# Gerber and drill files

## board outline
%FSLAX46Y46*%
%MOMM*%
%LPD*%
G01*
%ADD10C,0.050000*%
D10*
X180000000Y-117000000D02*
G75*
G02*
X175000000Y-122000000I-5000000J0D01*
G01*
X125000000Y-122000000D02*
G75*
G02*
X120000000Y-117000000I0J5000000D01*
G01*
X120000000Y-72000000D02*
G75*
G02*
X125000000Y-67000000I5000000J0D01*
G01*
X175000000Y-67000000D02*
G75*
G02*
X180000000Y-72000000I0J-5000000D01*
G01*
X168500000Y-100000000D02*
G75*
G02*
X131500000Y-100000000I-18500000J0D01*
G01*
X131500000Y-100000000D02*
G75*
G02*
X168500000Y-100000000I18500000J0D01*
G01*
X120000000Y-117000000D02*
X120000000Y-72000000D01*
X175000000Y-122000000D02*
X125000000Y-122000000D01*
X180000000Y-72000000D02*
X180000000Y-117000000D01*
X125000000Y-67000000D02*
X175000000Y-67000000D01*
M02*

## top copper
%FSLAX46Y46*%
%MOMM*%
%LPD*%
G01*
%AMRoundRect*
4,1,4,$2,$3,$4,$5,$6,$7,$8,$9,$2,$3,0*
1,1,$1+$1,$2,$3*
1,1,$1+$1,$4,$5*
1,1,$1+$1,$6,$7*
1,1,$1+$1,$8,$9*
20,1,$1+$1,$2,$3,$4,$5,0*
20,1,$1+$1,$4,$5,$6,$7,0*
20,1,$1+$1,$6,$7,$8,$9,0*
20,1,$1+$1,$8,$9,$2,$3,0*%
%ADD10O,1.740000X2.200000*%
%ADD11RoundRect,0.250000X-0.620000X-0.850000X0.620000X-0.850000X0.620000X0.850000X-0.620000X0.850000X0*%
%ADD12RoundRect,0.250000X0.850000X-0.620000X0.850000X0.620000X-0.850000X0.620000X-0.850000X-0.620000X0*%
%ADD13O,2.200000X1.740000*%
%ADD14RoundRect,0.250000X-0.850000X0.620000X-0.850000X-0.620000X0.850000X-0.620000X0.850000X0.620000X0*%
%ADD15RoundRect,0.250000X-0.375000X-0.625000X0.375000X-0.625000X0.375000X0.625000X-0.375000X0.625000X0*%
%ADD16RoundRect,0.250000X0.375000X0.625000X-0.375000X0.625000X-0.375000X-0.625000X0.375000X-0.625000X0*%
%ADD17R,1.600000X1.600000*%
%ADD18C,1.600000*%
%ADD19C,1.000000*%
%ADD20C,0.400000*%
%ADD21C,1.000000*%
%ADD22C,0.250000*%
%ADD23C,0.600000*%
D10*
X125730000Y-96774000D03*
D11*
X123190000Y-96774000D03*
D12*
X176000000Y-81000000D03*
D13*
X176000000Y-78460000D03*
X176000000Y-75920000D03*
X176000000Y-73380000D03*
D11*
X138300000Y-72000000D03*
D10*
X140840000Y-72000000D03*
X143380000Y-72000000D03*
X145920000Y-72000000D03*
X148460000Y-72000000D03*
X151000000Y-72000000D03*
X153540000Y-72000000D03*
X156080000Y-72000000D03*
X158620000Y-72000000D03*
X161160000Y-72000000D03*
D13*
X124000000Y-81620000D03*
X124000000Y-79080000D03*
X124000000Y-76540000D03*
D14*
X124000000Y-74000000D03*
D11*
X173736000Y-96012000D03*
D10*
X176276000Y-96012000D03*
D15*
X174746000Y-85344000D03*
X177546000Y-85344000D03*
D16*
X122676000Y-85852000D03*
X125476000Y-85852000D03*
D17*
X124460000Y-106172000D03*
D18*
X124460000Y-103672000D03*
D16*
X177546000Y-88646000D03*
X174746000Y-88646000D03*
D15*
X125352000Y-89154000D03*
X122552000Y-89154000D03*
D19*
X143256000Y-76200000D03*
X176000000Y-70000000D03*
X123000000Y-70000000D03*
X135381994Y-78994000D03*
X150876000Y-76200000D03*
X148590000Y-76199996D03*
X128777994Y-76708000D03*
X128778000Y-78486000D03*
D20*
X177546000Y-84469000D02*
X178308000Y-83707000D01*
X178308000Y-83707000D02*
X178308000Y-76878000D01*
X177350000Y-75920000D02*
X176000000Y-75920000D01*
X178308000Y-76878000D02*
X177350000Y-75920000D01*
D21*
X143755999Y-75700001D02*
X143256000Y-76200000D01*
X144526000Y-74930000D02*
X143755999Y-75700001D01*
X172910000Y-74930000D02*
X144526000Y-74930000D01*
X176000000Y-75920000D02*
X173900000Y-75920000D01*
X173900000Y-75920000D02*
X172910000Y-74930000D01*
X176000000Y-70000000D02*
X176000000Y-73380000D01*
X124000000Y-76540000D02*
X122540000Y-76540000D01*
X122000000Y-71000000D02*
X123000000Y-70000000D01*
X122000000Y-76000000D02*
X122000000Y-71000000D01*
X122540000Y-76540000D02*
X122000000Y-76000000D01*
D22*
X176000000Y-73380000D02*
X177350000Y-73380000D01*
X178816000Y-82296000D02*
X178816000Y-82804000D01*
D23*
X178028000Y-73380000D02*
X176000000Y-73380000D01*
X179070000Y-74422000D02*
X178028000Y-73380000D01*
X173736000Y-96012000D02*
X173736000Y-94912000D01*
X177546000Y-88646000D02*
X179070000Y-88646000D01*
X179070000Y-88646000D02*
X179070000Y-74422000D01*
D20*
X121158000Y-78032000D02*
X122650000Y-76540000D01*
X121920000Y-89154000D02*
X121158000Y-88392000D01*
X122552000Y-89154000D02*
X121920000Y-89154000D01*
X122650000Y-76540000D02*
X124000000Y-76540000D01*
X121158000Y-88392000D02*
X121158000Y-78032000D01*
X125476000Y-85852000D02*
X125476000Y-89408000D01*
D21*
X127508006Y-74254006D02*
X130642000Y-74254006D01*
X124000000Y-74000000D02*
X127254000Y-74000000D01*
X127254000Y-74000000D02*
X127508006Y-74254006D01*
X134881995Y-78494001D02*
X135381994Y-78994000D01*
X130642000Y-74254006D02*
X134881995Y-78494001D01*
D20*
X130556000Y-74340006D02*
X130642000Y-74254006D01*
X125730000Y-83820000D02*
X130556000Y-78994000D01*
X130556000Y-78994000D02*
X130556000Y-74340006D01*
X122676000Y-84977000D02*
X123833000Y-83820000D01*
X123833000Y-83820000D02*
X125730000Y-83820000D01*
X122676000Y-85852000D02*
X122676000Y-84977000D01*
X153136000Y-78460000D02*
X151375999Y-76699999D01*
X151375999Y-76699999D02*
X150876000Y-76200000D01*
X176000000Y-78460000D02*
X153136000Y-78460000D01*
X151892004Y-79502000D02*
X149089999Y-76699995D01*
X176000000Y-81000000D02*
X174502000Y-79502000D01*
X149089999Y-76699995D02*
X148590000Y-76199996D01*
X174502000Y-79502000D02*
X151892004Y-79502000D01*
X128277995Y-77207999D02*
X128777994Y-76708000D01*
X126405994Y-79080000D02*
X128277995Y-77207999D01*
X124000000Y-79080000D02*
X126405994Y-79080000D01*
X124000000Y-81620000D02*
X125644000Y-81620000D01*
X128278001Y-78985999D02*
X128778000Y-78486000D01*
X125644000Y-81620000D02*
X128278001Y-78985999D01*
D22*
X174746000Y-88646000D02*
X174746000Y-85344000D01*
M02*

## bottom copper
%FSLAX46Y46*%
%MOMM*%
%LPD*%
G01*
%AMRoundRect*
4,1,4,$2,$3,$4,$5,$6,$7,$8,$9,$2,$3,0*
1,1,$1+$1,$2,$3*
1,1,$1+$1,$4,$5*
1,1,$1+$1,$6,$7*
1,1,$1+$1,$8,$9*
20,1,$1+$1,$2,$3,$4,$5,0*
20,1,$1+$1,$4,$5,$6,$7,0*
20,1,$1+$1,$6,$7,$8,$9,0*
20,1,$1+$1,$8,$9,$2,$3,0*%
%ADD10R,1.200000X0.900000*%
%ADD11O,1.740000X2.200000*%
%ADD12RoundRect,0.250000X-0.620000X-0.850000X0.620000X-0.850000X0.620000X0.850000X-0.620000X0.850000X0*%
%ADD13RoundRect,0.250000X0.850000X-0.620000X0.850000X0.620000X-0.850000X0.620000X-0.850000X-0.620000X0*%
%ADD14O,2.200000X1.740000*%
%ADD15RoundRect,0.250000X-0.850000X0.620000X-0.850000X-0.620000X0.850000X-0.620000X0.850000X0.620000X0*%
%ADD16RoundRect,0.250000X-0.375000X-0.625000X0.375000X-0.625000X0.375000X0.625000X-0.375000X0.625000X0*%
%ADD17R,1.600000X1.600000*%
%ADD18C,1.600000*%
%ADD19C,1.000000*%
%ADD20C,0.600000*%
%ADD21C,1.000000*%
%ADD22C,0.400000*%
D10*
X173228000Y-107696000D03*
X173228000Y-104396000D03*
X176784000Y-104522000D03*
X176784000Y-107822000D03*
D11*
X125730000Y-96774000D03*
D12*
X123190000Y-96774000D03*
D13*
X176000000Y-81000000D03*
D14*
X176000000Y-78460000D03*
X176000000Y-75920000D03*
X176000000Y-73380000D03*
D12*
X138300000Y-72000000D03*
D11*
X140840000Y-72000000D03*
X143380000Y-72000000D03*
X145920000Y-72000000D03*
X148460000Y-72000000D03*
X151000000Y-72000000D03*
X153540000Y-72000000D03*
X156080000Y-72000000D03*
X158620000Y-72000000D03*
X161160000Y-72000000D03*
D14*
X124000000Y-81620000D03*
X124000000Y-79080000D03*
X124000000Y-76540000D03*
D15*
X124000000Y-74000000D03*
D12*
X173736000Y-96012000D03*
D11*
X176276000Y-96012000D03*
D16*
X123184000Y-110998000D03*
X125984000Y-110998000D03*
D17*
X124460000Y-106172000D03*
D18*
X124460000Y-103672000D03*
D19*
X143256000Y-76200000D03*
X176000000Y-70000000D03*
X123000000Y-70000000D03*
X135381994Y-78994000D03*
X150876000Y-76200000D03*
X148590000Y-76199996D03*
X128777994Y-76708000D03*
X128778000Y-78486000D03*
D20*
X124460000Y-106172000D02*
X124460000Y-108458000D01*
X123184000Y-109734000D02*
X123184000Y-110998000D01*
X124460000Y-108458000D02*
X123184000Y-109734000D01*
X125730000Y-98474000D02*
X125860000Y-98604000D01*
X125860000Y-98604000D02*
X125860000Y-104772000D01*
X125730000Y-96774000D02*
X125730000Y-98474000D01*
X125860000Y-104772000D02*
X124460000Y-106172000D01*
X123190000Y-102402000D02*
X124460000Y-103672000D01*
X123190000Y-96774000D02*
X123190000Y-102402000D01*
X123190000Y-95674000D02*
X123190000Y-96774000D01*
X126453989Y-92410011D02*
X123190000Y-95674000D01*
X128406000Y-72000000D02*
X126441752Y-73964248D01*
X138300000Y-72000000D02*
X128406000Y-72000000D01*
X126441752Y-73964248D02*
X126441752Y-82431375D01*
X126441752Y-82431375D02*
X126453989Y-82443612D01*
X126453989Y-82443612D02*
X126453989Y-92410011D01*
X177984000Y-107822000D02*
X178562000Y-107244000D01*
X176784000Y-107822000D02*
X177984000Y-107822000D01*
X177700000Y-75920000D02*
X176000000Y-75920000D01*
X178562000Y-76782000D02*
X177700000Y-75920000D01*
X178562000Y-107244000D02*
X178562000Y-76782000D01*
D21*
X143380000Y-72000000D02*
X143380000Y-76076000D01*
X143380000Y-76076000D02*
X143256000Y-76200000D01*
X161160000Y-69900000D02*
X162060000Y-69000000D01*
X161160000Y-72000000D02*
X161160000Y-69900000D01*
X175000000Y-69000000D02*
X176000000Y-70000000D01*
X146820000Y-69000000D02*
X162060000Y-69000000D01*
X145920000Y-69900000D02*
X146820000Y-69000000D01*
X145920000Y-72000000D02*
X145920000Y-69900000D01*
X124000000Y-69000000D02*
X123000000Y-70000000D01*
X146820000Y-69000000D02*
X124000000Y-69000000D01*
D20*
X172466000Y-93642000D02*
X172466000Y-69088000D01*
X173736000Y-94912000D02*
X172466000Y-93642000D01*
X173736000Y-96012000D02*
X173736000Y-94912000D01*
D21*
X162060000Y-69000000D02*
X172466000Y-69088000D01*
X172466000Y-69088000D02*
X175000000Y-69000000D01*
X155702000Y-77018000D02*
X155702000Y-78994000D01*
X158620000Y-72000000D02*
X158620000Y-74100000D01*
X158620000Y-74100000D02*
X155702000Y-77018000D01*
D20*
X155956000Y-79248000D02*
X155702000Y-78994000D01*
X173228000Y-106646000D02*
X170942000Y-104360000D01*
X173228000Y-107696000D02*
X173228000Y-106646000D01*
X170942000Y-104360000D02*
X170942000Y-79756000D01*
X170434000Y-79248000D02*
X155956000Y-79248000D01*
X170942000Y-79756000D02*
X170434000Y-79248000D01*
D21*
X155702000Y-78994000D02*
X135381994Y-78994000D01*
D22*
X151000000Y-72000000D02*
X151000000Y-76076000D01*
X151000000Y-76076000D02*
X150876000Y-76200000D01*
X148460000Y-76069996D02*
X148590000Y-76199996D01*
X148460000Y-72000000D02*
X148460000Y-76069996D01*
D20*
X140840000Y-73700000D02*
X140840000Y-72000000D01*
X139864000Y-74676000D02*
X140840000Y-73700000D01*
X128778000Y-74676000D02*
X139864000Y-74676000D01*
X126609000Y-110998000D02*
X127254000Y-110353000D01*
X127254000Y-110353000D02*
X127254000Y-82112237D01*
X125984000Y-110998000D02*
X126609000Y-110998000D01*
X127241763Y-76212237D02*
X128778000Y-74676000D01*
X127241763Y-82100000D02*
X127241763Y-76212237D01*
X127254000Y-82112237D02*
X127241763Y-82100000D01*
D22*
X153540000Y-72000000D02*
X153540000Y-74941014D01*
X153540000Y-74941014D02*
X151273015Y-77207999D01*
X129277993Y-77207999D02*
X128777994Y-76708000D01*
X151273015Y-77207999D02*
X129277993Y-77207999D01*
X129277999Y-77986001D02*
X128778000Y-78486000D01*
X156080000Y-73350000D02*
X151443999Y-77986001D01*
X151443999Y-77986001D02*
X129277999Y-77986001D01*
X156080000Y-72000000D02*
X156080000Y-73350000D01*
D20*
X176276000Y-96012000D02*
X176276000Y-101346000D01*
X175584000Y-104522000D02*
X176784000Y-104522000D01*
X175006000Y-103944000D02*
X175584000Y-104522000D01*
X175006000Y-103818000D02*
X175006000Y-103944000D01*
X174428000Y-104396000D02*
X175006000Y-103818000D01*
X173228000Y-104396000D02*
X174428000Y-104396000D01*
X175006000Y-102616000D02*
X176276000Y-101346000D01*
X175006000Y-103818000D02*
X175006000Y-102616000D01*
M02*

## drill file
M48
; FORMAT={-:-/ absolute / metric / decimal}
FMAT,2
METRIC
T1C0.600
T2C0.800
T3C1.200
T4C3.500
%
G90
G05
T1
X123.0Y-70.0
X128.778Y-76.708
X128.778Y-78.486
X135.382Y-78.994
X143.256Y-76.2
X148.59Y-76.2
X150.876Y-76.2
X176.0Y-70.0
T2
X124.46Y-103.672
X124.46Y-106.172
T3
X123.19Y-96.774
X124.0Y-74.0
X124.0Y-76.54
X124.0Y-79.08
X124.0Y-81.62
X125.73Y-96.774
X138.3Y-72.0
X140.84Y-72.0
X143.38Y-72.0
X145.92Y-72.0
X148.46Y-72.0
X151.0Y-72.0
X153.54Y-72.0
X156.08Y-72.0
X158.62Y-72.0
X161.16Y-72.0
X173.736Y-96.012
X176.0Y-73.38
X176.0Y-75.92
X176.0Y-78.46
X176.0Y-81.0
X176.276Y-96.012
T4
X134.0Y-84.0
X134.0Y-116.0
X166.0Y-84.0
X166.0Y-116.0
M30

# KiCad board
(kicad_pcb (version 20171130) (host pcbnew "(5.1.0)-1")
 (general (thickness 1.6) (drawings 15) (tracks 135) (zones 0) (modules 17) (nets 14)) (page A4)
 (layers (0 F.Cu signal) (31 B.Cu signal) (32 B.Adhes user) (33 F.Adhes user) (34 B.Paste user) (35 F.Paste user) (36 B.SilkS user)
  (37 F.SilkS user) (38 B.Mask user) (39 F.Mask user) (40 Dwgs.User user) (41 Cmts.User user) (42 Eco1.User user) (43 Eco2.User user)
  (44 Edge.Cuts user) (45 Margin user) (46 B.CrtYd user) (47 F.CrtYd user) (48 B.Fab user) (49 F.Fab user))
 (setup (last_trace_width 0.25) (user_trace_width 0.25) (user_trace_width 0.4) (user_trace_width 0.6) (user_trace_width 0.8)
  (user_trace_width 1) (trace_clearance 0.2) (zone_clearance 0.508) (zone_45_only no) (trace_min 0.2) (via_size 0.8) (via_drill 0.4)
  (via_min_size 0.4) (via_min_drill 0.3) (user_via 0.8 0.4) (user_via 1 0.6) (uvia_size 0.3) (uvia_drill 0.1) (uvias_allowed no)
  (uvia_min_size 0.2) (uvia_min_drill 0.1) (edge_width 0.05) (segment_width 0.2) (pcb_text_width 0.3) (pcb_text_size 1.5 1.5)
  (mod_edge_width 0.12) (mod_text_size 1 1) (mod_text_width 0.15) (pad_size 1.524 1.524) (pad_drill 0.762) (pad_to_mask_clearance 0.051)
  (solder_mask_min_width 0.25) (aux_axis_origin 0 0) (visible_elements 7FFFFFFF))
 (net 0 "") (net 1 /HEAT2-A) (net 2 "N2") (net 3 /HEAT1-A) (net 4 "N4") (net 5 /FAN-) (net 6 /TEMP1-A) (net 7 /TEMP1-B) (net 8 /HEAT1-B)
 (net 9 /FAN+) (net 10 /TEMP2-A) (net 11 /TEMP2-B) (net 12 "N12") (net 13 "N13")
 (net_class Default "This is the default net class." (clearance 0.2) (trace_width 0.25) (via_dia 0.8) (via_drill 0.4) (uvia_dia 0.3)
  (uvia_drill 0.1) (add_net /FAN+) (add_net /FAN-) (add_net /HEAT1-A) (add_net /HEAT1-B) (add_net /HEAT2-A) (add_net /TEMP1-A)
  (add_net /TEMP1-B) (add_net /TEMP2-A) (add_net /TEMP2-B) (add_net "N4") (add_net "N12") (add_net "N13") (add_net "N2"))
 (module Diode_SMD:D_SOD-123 (layer B.Cu) (at 173.228 106.046 270)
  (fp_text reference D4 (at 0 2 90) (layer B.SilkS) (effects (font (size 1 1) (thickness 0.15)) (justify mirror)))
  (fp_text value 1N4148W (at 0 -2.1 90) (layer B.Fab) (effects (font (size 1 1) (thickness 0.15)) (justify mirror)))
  (pad 2 smd rect (at 1.65 0 270) (size 0.9 1.2) (layers B.Cu B.Paste B.Mask) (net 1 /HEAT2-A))
  (pad 1 smd rect (at -1.65 0 270) (size 0.9 1.2) (layers B.Cu B.Paste B.Mask) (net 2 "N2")))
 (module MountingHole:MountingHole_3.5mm (layer F.Cu) (at 134 116)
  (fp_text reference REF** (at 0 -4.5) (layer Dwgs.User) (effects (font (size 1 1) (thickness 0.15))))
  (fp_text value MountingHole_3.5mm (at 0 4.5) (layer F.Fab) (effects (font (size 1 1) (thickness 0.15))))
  (pad 1 np_thru_hole circle (at 0 0) (size 3.5 3.5) (drill 3.5) (layers *.Cu *.Mask)))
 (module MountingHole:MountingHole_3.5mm (layer F.Cu) (at 166 116)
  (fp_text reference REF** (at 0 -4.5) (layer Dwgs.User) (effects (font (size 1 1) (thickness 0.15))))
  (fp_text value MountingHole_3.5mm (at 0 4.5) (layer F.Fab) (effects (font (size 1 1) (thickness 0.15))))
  (pad 1 np_thru_hole circle (at 0 0) (size 3.5 3.5) (drill 3.5) (layers *.Cu *.Mask)))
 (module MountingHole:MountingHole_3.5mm (layer F.Cu) (at 166 84)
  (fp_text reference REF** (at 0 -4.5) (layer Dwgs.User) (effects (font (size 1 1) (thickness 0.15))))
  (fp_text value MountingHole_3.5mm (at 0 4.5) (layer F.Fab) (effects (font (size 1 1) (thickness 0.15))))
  (pad 1 np_thru_hole circle (at 0 0) (size 3.5 3.5) (drill 3.5) (layers *.Cu *.Mask)))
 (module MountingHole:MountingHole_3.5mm (layer F.Cu) (at 134 84)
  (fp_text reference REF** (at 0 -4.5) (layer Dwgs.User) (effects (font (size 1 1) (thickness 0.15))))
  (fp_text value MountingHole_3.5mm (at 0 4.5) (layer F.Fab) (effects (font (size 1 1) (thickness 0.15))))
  (pad 1 np_thru_hole circle (at 0 0) (size 3.5 3.5) (drill 3.5) (layers *.Cu *.Mask)))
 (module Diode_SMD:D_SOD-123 (layer B.Cu) (at 176.784 106.172 270)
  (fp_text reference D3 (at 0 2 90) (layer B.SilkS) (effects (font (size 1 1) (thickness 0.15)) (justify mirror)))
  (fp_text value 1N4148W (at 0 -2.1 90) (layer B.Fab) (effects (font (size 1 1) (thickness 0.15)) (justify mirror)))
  (pad 1 smd rect (at -1.65 0 270) (size 0.9 1.2) (layers B.Cu B.Paste B.Mask) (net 2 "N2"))
  (pad 2 smd rect (at 1.65 0 270) (size 0.9 1.2) (layers B.Cu B.Paste B.Mask) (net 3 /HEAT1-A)))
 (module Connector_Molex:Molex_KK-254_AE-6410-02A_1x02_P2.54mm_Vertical (layer F.Cu) (at 123.19 96.774)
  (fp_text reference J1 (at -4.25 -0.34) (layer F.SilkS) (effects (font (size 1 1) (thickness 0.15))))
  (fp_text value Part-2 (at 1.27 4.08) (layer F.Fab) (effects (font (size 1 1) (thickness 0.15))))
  (pad 2 thru_hole oval (at 2.54 0) (size 1.74 2.2) (drill 1.2) (layers *.Cu *.Mask) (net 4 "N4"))
  (pad 1 thru_hole roundrect (at 0 0) (size 1.74 2.2) (drill 1.2) (layers *.Cu *.Mask) (roundrect_rratio 0.143678) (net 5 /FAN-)))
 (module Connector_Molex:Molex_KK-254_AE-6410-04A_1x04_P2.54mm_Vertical (layer B.Cu) (at 176 81 90)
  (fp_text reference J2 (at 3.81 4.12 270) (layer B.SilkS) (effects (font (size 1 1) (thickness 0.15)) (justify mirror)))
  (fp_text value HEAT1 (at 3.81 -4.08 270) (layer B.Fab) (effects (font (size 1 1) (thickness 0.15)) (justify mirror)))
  (pad 1 thru_hole roundrect (at 0 0 90) (size 1.74 2.2) (drill 1.2) (layers *.Cu *.Mask) (roundrect_rratio 0.143678) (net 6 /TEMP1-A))
  (pad 2 thru_hole oval (at 2.54 0 90) (size 1.74 2.2) (drill 1.2) (layers *.Cu *.Mask) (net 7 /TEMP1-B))
  (pad 3 thru_hole oval (at 5.08 0 90) (size 1.74 2.2) (drill 1.2) (layers *.Cu *.Mask) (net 3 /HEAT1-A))
  (pad 4 thru_hole oval (at 7.62 0 90) (size 1.74 2.2) (drill 1.2) (layers *.Cu *.Mask) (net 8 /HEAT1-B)))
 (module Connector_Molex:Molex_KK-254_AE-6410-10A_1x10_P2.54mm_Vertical (layer F.Cu) (at 138.3 72)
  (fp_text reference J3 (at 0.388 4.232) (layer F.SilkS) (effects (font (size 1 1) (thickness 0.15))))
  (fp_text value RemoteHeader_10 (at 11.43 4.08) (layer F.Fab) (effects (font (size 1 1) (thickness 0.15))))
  (pad 1 thru_hole roundrect (at 0 0) (size 1.74 2.2) (drill 1.2) (layers *.Cu *.Mask) (roundrect_rratio 0.143678) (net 5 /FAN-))
  (pad 2 thru_hole oval (at 2.54 0) (size 1.74 2.2) (drill 1.2) (layers *.Cu *.Mask) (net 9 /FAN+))
  (pad 3 thru_hole oval (at 5.08 0) (size 1.74 2.2) (drill 1.2) (layers *.Cu *.Mask) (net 3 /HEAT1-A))
  (pad 4 thru_hole oval (at 7.62 0) (size 1.74 2.2) (drill 1.2) (layers *.Cu *.Mask) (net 8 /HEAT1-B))
  (pad 5 thru_hole oval (at 10.16 0) (size 1.74 2.2) (drill 1.2) (layers *.Cu *.Mask) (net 6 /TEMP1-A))
  (pad 6 thru_hole oval (at 12.7 0) (size 1.74 2.2) (drill 1.2) (layers *.Cu *.Mask) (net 7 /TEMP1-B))
  (pad 7 thru_hole oval (at 15.24 0) (size 1.74 2.2) (drill 1.2) (layers *.Cu *.Mask) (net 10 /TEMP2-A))
  (pad 8 thru_hole oval (at 17.78 0) (size 1.74 2.2) (drill 1.2) (layers *.Cu *.Mask) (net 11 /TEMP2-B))
  (pad 9 thru_hole oval (at 20.32 0) (size 1.74 2.2) (drill 1.2) (layers *.Cu *.Mask) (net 1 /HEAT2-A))
  (pad 10 thru_hole oval (at 22.86 0) (size 1.74 2.2) (drill 1.2) (layers *.Cu *.Mask) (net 8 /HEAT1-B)))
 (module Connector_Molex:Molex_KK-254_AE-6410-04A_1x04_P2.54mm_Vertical (layer B.Cu) (at 124 74 270)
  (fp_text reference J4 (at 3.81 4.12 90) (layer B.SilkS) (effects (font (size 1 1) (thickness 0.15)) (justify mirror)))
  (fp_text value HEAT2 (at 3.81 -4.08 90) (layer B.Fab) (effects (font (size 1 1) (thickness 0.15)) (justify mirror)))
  (pad 4 thru_hole oval (at 7.62 0 270) (size 1.74 2.2) (drill 1.2) (layers *.Cu *.Mask) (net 11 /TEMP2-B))
  (pad 3 thru_hole oval (at 5.08 0 270) (size 1.74 2.2) (drill 1.2) (layers *.Cu *.Mask) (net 10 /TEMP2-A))
  (pad 2 thru_hole oval (at 2.54 0 270) (size 1.74 2.2) (drill 1.2) (layers *.Cu *.Mask) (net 8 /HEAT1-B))
  (pad 1 thru_hole roundrect (at 0 0 270) (size 1.74 2.2) (drill 1.2) (layers *.Cu *.Mask) (roundrect_rratio 0.143678) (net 1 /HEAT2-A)))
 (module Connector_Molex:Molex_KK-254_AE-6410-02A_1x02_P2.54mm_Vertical (layer F.Cu) (at 173.736 96.012)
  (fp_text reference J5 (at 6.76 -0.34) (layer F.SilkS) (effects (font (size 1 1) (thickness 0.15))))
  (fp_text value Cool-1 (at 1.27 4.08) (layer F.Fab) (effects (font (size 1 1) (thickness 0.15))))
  (pad 1 thru_hole roundrect (at 0 0) (size 1.74 2.2) (drill 1.2) (layers *.Cu *.Mask) (roundrect_rratio 0.143678) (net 8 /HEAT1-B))
  (pad 2 thru_hole oval (at 2.54 0) (size 1.74 2.2) (drill 1.2) (layers *.Cu *.Mask) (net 2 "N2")))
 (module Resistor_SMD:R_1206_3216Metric (layer F.Cu) (at 176.146 85.344)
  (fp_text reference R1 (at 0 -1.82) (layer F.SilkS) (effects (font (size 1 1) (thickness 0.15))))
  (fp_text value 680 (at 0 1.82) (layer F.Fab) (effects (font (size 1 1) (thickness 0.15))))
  (pad 1 smd roundrect (at -1.4 0) (size 1.25 1.75) (layers F.Cu F.Paste F.Mask) (roundrect_rratio 0.2) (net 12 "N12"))
  (pad 2 smd roundrect (at 1.4 0) (size 1.25 1.75) (layers F.Cu F.Paste F.Mask) (roundrect_rratio 0.2) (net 3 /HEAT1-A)))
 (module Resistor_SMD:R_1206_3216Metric (layer B.Cu) (at 124.584 110.998)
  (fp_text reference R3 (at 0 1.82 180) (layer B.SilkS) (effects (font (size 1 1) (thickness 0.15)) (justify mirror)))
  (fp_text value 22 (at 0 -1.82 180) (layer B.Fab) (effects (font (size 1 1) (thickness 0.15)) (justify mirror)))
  (pad 1 smd roundrect (at -1.4 0) (size 1.25 1.75) (layers B.Cu B.Paste B.Mask) (roundrect_rratio 0.2) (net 4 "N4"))
  (pad 2 smd roundrect (at 1.4 0) (size 1.25 1.75) (layers B.Cu B.Paste B.Mask) (roundrect_rratio 0.2) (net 9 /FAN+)))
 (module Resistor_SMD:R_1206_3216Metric (layer F.Cu) (at 124.076 85.852 180)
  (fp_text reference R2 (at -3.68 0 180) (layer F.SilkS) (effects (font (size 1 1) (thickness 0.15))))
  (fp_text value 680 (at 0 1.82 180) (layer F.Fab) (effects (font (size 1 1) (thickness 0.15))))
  (pad 2 smd roundrect (at 1.4 0 180) (size 1.25 1.75) (layers F.Cu F.Paste F.Mask) (roundrect_rratio 0.2) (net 1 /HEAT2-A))
  (pad 1 smd roundrect (at -1.4 0 180) (size 1.25 1.75) (layers F.Cu F.Paste F.Mask) (roundrect_rratio 0.2) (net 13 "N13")))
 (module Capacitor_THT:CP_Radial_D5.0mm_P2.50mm (layer F.Cu) (at 124.46 106.172 90)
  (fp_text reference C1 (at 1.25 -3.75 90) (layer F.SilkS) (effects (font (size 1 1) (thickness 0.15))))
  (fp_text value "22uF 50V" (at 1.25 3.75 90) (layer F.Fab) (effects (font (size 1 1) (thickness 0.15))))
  (pad 1 thru_hole rect (at 0 0 90) (size 1.6 1.6) (drill 0.8) (layers *.Cu *.Mask) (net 4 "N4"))
  (pad 2 thru_hole circle (at 2.5 0 90) (size 1.6 1.6) (drill 0.8) (layers *.Cu *.Mask) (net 5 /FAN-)))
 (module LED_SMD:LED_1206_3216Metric (layer F.Cu) (at 176.146 88.646 180)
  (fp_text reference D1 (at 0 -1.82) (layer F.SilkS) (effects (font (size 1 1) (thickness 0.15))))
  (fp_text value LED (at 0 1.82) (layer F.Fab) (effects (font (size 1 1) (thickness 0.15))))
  (pad 1 smd roundrect (at -1.4 0 180) (size 1.25 1.75) (layers F.Cu F.Paste F.Mask) (roundrect_rratio 0.2) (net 8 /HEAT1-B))
  (pad 2 smd roundrect (at 1.4 0 180) (size 1.25 1.75) (layers F.Cu F.Paste F.Mask) (roundrect_rratio 0.2) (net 12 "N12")))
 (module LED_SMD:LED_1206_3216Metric (layer F.Cu) (at 123.952 89.154)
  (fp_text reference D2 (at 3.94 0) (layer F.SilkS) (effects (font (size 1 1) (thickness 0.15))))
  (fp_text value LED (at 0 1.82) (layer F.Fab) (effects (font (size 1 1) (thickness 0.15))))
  (pad 2 smd roundrect (at 1.4 0) (size 1.25 1.75) (layers F.Cu F.Paste F.Mask) (roundrect_rratio 0.2) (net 13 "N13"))
  (pad 1 smd roundrect (at -1.4 0) (size 1.25 1.75) (layers F.Cu F.Paste F.Mask) (roundrect_rratio 0.2) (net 8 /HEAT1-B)))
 (gr_arc (start 175 117) (end 175 122) (angle -90) (layer Edge.Cuts) (width 0.05))
 (gr_arc (start 125 117) (end 120 117) (angle -90) (layer Edge.Cuts) (width 0.05))
 (gr_arc (start 125 72) (end 125 67) (angle -90) (layer Edge.Cuts) (width 0.05))
 (gr_arc (start 175 72) (end 180 72) (angle -90) (layer Edge.Cuts) (width 0.05))
 (gr_circle (center 150 100) (end 168.5 100) (layer Edge.Cuts) (width 0.05))
 (gr_line (start 120 117) (end 120 72) (layer Edge.Cuts) (width 0.05))
 (gr_line (start 175 122) (end 125 122) (layer Edge.Cuts) (width 0.05))
 (gr_line (start 180 72) (end 180 117) (layer Edge.Cuts) (width 0.05))
 (gr_line (start 125 67) (end 175 67) (layer Edge.Cuts) (width 0.05))
 (segment (start 124.46 106.172) (end 124.46 108.458) (width 0.6) (layer B.Cu) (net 4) (status 10))
 (segment (start 123.184 109.734) (end 123.184 110.998) (width 0.6) (layer B.Cu) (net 4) (status 20))
 (segment (start 124.46 108.458) (end 123.184 109.734) (width 0.6) (layer B.Cu) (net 4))
 (segment (start 125.73 98.474) (end 125.86 98.604) (width 0.6) (layer B.Cu) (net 4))
 (segment (start 125.86 98.604) (end 125.86 104.772) (width 0.6) (layer B.Cu) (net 4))
 (segment (start 125.73 96.774) (end 125.73 98.474) (width 0.6) (layer B.Cu) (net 4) (status 10))
 (segment (start 125.86 104.772) (end 124.46 106.172) (width 0.6) (layer B.Cu) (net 4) (status 20))
 (segment (start 123.19 102.402) (end 124.46 103.672) (width 0.6) (layer B.Cu) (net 5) (status 20))
 (segment (start 123.19 96.774) (end 123.19 102.402) (width 0.6) (layer B.Cu) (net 5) (status 10))
 (segment (start 123.19 95.674) (end 123.19 96.774) (width 0.6) (layer B.Cu) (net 5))
 (segment (start 126.453989 92.410011) (end 123.19 95.674) (width 0.6) (layer B.Cu) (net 5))
 (segment (start 128.406 72) (end 126.441752 73.964248) (width 0.6) (layer B.Cu) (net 5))
 (segment (start 138.3 72) (end 128.406 72) (width 0.6) (layer B.Cu) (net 5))
 (segment (start 126.441752 73.964248) (end 126.441752 82.431375) (width 0.6) (layer B.Cu) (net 5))
 (segment (start 126.441752 82.431375) (end 126.453989 82.443612) (width 0.6) (layer B.Cu) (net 5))
 (segment (start 126.453989 82.443612) (end 126.453989 92.410011) (width 0.6) (layer B.Cu) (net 5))
 (segment (start 177.546 84.469) (end 178.308 83.707) (width 0.4) (layer F.Cu) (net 3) (status 1000010))
 (segment (start 178.308 83.707) (end 178.308 76.878) (width 0.4) (layer F.Cu) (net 3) (status 1000000))
 (segment (start 177.35 75.92) (end 176 75.92) (width 0.4) (layer F.Cu) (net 3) (status 1000020))
 (segment (start 178.308 76.878) (end 177.35 75.92) (width 0.4) (layer F.Cu) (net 3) (status 1000000))
 (segment (start 177.984 107.822) (end 178.562 107.244) (width 0.6) (layer B.Cu) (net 3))
 (segment (start 176.784 107.822) (end 177.984 107.822) (width 0.6) (layer B.Cu) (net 3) (status 10))
 (segment (start 177.7 75.92) (end 176 75.92) (width 0.6) (layer B.Cu) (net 3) (status 20))
 (segment (start 178.562 76.782) (end 177.7 75.92) (width 0.6) (layer B.Cu) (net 3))
 (segment (start 178.562 107.244) (end 178.562 76.782) (width 0.6) (layer B.Cu) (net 3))
 (via (at 143.256 76.2) (size 1) (drill 0.6) (layers F.Cu B.Cu) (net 3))
 (segment (start 143.38 72) (end 143.38 76.076) (width 1) (layer B.Cu) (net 3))
 (segment (start 143.38 76.076) (end 143.256 76.2) (width 1) (layer B.Cu) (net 3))
 (segment (start 143.755999 75.700001) (end 143.256 76.2) (width 1) (layer F.Cu) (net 3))
 (segment (start 144.526 74.93) (end 143.755999 75.700001) (width 1) (layer F.Cu) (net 3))
 (segment (start 172.91 74.93) (end 144.526 74.93) (width 1) (layer F.Cu) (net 3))
 (segment (start 176 75.92) (end 173.9 75.92) (width 1) (layer F.Cu) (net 3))
 (segment (start 173.9 75.92) (end 172.91 74.93) (width 1) (layer F.Cu) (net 3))
 (segment (start 161.16 69.9) (end 162.06 69) (width 1) (layer B.Cu) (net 8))
 (segment (start 161.16 72) (end 161.16 69.9) (width 1) (layer B.Cu) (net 8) (status 10))
 (via (at 176 70) (size 1) (drill 0.6) (layers F.Cu B.Cu) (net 8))
 (segment (start 175 69) (end 176 70) (width 1) (layer B.Cu) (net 8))
 (segment (start 176 70) (end 176 73.38) (width 1) (layer F.Cu) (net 8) (status 20))
 (segment (start 146.82 69) (end 162.06 69) (width 1) (layer B.Cu) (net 8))
 (segment (start 145.92 69.9) (end 146.82 69) (width 1) (layer B.Cu) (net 8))
 (segment (start 145.92 72) (end 145.92 69.9) (width 1) (layer B.Cu) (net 8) (status 10))
 (segment (start 124 76.54) (end 122.54 76.54) (width 1) (layer F.Cu) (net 8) (status 10))
 (segment (start 124 69) (end 123 70) (width 1) (layer B.Cu) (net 8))
 (segment (start 146.82 69) (end 124 69) (width 1) (layer B.Cu) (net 8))
 (via (at 123 70) (size 1) (drill 0.6) (layers F.Cu B.Cu) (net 8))
 (segment (start 122 71) (end 123 70) (width 1) (layer F.Cu) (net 8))
 (segment (start 122 76) (end 122 71) (width 1) (layer F.Cu) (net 8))
 (segment (start 122.54 76.54) (end 122 76) (width 1) (layer F.Cu) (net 8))
 (segment (start 176 73.38) (end 177.35 73.38) (width 0.25) (layer F.Cu) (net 8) (status 10))
 (segment (start 178.816 82.296) (end 178.816 82.804) (width 0.25) (layer F.Cu) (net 8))
 (segment (start 178.028 73.38) (end 176 73.38) (width 0.6) (layer F.Cu) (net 8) (status 20))
 (segment (start 179.07 74.422) (end 178.028 73.38) (width 0.6) (layer F.Cu) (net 8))
 (segment (start 173.736 96.012) (end 173.736 94.912) (width 0.6) (layer F.Cu) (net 8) (status 30))
 (segment (start 177.546 88.646) (end 179.07 88.646) (width 0.6) (layer F.Cu) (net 8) (status 10))
 (segment (start 179.07 88.646) (end 179.07 74.422) (width 0.6) (layer F.Cu) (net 8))
 (segment (start 172.466 93.642) (end 172.466 69.088) (width 0.6) (layer B.Cu) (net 8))
 (segment (start 173.736 94.912) (end 172.466 93.642) (width 0.6) (layer B.Cu) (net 8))
 (segment (start 173.736 96.012) (end 173.736 94.912) (width 0.6) (layer B.Cu) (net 8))
 (segment (start 162.06 69) (end 172.466 69.088) (width 1) (layer B.Cu) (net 8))
 (segment (start 172.466 69.088) (end 175 69) (width 1) (layer B.Cu) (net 8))
 (segment (start 121.158 78.032) (end 122.65 76.54) (width 0.4) (layer F.Cu) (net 8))
 (segment (start 121.92 89.154) (end 121.158 88.392) (width 0.4) (layer F.Cu) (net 8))
 (segment (start 122.552 89.154) (end 121.92 89.154) (width 0.4) (layer F.Cu) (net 8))
 (segment (start 122.65 76.54) (end 124 76.54) (width 0.4) (layer F.Cu) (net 8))
 (segment (start 121.158 88.392) (end 121.158 78.032) (width 0.4) (layer F.Cu) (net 8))
 (segment (start 125.476 85.852) (end 125.476 89.408) (width 0.4) (layer F.Cu) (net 13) (status 30))
 (segment (start 155.702 77.018) (end 155.702 78.994) (width 1) (layer B.Cu) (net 1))
 (segment (start 158.62 72) (end 158.62 74.1) (width 1) (layer B.Cu) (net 1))
 (segment (start 158.62 74.1) (end 155.702 77.018) (width 1) (layer B.Cu) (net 1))
 (segment (start 155.956 79.248) (end 155.702 78.994) (width 0.6) (layer B.Cu) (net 1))
 (segment (start 173.228 106.646) (end 170.942 104.36) (width 0.6) (layer B.Cu) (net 1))
 (segment (start 173.228 107.696) (end 173.228 106.646) (width 0.6) (layer B.Cu) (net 1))
 (segment (start 170.942 104.36) (end 170.942 79.756) (width 0.6) (layer B.Cu) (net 1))
 (segment (start 170.434 79.248) (end 155.956 79.248) (width 0.6) (layer B.Cu) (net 1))
 (segment (start 170.942 79.756) (end 170.434 79.248) (width 0.6) (layer B.Cu) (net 1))
 (segment (start 155.702 78.994) (end 135.381994 78.994) (width 1) (layer B.Cu) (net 1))
 (via (at 135.381994 78.994) (size 1) (drill 0.6) (layers F.Cu B.Cu) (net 1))
 (segment (start 127.508006 74.254006) (end 130.642 74.254006) (width 1) (layer F.Cu) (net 1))
 (segment (start 124 74) (end 127.254 74) (width 1) (layer F.Cu) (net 1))
 (segment (start 127.254 74) (end 127.508006 74.254006) (width 1) (layer F.Cu) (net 1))
 (segment (start 134.881995 78.494001) (end 135.381994 78.994) (width 1) (layer F.Cu) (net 1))
 (segment (start 130.642 74.254006) (end 134.881995 78.494001) (width 1) (layer F.Cu) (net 1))
 (segment (start 130.556 74.340006) (end 130.642 74.254006) (width 0.4) (layer F.Cu) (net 1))
 (segment (start 125.73 83.82) (end 130.556 78.994) (width 0.4) (layer F.Cu) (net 1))
 (segment (start 130.556 78.994) (end 130.556 74.340006) (width 0.4) (layer F.Cu) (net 1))
 (segment (start 122.676 84.977) (end 123.833 83.82) (width 0.4) (layer F.Cu) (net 1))
 (segment (start 123.833 83.82) (end 125.73 83.82) (width 0.4) (layer F.Cu) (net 1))
 (segment (start 122.676 85.852) (end 122.676 84.977) (width 0.4) (layer F.Cu) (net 1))
 (segment (start 151 72) (end 151 76.076) (width 0.4) (layer B.Cu) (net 7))
 (segment (start 153.136 78.46) (end 151.375999 76.699999) (width 0.4) (layer F.Cu) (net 7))
 (segment (start 151.375999 76.699999) (end 150.876 76.2) (width 0.4) (layer F.Cu) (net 7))
 (via (at 150.876 76.2) (size 1) (drill 0.6) (layers F.Cu B.Cu) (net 7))
 (segment (start 151 76.076) (end 150.876 76.2) (width 0.4) (layer B.Cu) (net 7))
 (segment (start 176 78.46) (end 153.136 78.46) (width 0.4) (layer F.Cu) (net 7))
 (via (at 148.59 76.199996) (size 1) (drill 0.6) (layers F.Cu B.Cu) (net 6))
 (segment (start 148.46 76.069996) (end 148.59 76.199996) (width 0.4) (layer B.Cu) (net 6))
 (segment (start 148.46 72) (end 148.46 76.069996) (width 0.4) (layer B.Cu) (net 6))
 (segment (start 151.892004 79.502) (end 149.089999 76.699995) (width 0.4) (layer F.Cu) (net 6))
 (segment (start 176 81) (end 174.502 79.502) (width 0.4) (layer F.Cu) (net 6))
 (segment (start 149.089999 76.699995) (end 148.59 76.199996) (width 0.4) (layer F.Cu) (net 6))
 (segment (start 174.502 79.502) (end 151.892004 79.502) (width 0.4) (layer F.Cu) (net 6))
 (segment (start 140.84 73.7) (end 140.84 72) (width 0.6) (layer B.Cu) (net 9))
 (segment (start 139.864 74.676) (end 140.84 73.7) (width 0.6) (layer B.Cu) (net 9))
 (segment (start 128.778 74.676) (end 139.864 74.676) (width 0.6) (layer B.Cu) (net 9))
 (segment (start 126.609 110.998) (end 127.254 110.353) (width 0.6) (layer B.Cu) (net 9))
 (segment (start 127.254 110.353) (end 127.254 82.112237) (width 0.6) (layer B.Cu) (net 9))
 (segment (start 125.984 110.998) (end 126.609 110.998) (width 0.6) (layer B.Cu) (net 9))
 (segment (start 127.241763 76.212237) (end 128.778 74.676) (width 0.6) (layer B.Cu) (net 9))
 (segment (start 127.241763 82.1) (end 127.241763 76.212237) (width 0.6) (layer B.Cu) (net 9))
 (segment (start 127.254 82.112237) (end 127.241763 82.1) (width 0.6) (layer B.Cu) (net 9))
 (via (at 128.777994 76.708) (size 1) (drill 0.6) (layers F.Cu B.Cu) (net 10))
 (segment (start 153.54 72) (end 153.54 74.941014) (width 0.4) (layer B.Cu) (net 10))
 (segment (start 128.277995 77.207999) (end 128.777994 76.708) (width 0.4) (layer F.Cu) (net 10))
 (segment (start 153.54 74.941014) (end 151.273015 77.207999) (width 0.4) (layer B.Cu) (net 10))
 (segment (start 129.277993 77.207999) (end 128.777994 76.708) (width 0.4) (layer B.Cu) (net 10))
 (segment (start 151.273015 77.207999) (end 129.277993 77.207999) (width 0.4) (layer B.Cu) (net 10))
 (segment (start 126.405994 79.08) (end 128.277995 77.207999) (width 0.4) (layer F.Cu) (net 10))
 (segment (start 124 79.08) (end 126.405994 79.08) (width 0.4) (layer F.Cu) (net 10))
 (segment (start 129.277999 77.986001) (end 128.778 78.486) (width 0.4) (layer B.Cu) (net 11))
 (segment (start 124 81.62) (end 125.644 81.62) (width 0.4) (layer F.Cu) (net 11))
 (segment (start 156.08 73.35) (end 151.443999 77.986001) (width 0.4) (layer B.Cu) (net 11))
 (via (at 128.778 78.486) (size 1) (drill 0.6) (layers F.Cu B.Cu) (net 11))
 (segment (start 128.278001 78.985999) (end 128.778 78.486) (width 0.4) (layer F.Cu) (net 11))
 (segment (start 151.443999 77.986001) (end 129.277999 77.986001) (width 0.4) (layer B.Cu) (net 11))
 (segment (start 125.644 81.62) (end 128.278001 78.985999) (width 0.4) (layer F.Cu) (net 11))
 (segment (start 156.08 72) (end 156.08 73.35) (width 0.4) (layer B.Cu) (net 11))
 (segment (start 174.746 88.646) (end 174.746 85.344) (width 0.25) (layer F.Cu) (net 12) (status 30))
 (segment (start 176.276 96.012) (end 176.276 101.346) (width 0.6) (layer B.Cu) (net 2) (status 10))
 (segment (start 175.584 104.522) (end 176.784 104.522) (width 0.6) (layer B.Cu) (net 2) (status 20))
 (segment (start 175.006 103.944) (end 175.584 104.522) (width 0.6) (layer B.Cu) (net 2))
 (segment (start 175.006 103.818) (end 175.006 103.944) (width 0.6) (layer B.Cu) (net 2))
 (segment (start 174.428 104.396) (end 175.006 103.818) (width 0.6) (layer B.Cu) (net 2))
 (segment (start 173.228 104.396) (end 174.428 104.396) (width 0.6) (layer B.Cu) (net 2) (status 10))
 (segment (start 175.006 102.616) (end 176.276 101.346) (width 0.6) (layer B.Cu) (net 2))
 (segment (start 175.006 103.818) (end 175.006 102.616) (width 0.6) (layer B.Cu) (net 2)))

